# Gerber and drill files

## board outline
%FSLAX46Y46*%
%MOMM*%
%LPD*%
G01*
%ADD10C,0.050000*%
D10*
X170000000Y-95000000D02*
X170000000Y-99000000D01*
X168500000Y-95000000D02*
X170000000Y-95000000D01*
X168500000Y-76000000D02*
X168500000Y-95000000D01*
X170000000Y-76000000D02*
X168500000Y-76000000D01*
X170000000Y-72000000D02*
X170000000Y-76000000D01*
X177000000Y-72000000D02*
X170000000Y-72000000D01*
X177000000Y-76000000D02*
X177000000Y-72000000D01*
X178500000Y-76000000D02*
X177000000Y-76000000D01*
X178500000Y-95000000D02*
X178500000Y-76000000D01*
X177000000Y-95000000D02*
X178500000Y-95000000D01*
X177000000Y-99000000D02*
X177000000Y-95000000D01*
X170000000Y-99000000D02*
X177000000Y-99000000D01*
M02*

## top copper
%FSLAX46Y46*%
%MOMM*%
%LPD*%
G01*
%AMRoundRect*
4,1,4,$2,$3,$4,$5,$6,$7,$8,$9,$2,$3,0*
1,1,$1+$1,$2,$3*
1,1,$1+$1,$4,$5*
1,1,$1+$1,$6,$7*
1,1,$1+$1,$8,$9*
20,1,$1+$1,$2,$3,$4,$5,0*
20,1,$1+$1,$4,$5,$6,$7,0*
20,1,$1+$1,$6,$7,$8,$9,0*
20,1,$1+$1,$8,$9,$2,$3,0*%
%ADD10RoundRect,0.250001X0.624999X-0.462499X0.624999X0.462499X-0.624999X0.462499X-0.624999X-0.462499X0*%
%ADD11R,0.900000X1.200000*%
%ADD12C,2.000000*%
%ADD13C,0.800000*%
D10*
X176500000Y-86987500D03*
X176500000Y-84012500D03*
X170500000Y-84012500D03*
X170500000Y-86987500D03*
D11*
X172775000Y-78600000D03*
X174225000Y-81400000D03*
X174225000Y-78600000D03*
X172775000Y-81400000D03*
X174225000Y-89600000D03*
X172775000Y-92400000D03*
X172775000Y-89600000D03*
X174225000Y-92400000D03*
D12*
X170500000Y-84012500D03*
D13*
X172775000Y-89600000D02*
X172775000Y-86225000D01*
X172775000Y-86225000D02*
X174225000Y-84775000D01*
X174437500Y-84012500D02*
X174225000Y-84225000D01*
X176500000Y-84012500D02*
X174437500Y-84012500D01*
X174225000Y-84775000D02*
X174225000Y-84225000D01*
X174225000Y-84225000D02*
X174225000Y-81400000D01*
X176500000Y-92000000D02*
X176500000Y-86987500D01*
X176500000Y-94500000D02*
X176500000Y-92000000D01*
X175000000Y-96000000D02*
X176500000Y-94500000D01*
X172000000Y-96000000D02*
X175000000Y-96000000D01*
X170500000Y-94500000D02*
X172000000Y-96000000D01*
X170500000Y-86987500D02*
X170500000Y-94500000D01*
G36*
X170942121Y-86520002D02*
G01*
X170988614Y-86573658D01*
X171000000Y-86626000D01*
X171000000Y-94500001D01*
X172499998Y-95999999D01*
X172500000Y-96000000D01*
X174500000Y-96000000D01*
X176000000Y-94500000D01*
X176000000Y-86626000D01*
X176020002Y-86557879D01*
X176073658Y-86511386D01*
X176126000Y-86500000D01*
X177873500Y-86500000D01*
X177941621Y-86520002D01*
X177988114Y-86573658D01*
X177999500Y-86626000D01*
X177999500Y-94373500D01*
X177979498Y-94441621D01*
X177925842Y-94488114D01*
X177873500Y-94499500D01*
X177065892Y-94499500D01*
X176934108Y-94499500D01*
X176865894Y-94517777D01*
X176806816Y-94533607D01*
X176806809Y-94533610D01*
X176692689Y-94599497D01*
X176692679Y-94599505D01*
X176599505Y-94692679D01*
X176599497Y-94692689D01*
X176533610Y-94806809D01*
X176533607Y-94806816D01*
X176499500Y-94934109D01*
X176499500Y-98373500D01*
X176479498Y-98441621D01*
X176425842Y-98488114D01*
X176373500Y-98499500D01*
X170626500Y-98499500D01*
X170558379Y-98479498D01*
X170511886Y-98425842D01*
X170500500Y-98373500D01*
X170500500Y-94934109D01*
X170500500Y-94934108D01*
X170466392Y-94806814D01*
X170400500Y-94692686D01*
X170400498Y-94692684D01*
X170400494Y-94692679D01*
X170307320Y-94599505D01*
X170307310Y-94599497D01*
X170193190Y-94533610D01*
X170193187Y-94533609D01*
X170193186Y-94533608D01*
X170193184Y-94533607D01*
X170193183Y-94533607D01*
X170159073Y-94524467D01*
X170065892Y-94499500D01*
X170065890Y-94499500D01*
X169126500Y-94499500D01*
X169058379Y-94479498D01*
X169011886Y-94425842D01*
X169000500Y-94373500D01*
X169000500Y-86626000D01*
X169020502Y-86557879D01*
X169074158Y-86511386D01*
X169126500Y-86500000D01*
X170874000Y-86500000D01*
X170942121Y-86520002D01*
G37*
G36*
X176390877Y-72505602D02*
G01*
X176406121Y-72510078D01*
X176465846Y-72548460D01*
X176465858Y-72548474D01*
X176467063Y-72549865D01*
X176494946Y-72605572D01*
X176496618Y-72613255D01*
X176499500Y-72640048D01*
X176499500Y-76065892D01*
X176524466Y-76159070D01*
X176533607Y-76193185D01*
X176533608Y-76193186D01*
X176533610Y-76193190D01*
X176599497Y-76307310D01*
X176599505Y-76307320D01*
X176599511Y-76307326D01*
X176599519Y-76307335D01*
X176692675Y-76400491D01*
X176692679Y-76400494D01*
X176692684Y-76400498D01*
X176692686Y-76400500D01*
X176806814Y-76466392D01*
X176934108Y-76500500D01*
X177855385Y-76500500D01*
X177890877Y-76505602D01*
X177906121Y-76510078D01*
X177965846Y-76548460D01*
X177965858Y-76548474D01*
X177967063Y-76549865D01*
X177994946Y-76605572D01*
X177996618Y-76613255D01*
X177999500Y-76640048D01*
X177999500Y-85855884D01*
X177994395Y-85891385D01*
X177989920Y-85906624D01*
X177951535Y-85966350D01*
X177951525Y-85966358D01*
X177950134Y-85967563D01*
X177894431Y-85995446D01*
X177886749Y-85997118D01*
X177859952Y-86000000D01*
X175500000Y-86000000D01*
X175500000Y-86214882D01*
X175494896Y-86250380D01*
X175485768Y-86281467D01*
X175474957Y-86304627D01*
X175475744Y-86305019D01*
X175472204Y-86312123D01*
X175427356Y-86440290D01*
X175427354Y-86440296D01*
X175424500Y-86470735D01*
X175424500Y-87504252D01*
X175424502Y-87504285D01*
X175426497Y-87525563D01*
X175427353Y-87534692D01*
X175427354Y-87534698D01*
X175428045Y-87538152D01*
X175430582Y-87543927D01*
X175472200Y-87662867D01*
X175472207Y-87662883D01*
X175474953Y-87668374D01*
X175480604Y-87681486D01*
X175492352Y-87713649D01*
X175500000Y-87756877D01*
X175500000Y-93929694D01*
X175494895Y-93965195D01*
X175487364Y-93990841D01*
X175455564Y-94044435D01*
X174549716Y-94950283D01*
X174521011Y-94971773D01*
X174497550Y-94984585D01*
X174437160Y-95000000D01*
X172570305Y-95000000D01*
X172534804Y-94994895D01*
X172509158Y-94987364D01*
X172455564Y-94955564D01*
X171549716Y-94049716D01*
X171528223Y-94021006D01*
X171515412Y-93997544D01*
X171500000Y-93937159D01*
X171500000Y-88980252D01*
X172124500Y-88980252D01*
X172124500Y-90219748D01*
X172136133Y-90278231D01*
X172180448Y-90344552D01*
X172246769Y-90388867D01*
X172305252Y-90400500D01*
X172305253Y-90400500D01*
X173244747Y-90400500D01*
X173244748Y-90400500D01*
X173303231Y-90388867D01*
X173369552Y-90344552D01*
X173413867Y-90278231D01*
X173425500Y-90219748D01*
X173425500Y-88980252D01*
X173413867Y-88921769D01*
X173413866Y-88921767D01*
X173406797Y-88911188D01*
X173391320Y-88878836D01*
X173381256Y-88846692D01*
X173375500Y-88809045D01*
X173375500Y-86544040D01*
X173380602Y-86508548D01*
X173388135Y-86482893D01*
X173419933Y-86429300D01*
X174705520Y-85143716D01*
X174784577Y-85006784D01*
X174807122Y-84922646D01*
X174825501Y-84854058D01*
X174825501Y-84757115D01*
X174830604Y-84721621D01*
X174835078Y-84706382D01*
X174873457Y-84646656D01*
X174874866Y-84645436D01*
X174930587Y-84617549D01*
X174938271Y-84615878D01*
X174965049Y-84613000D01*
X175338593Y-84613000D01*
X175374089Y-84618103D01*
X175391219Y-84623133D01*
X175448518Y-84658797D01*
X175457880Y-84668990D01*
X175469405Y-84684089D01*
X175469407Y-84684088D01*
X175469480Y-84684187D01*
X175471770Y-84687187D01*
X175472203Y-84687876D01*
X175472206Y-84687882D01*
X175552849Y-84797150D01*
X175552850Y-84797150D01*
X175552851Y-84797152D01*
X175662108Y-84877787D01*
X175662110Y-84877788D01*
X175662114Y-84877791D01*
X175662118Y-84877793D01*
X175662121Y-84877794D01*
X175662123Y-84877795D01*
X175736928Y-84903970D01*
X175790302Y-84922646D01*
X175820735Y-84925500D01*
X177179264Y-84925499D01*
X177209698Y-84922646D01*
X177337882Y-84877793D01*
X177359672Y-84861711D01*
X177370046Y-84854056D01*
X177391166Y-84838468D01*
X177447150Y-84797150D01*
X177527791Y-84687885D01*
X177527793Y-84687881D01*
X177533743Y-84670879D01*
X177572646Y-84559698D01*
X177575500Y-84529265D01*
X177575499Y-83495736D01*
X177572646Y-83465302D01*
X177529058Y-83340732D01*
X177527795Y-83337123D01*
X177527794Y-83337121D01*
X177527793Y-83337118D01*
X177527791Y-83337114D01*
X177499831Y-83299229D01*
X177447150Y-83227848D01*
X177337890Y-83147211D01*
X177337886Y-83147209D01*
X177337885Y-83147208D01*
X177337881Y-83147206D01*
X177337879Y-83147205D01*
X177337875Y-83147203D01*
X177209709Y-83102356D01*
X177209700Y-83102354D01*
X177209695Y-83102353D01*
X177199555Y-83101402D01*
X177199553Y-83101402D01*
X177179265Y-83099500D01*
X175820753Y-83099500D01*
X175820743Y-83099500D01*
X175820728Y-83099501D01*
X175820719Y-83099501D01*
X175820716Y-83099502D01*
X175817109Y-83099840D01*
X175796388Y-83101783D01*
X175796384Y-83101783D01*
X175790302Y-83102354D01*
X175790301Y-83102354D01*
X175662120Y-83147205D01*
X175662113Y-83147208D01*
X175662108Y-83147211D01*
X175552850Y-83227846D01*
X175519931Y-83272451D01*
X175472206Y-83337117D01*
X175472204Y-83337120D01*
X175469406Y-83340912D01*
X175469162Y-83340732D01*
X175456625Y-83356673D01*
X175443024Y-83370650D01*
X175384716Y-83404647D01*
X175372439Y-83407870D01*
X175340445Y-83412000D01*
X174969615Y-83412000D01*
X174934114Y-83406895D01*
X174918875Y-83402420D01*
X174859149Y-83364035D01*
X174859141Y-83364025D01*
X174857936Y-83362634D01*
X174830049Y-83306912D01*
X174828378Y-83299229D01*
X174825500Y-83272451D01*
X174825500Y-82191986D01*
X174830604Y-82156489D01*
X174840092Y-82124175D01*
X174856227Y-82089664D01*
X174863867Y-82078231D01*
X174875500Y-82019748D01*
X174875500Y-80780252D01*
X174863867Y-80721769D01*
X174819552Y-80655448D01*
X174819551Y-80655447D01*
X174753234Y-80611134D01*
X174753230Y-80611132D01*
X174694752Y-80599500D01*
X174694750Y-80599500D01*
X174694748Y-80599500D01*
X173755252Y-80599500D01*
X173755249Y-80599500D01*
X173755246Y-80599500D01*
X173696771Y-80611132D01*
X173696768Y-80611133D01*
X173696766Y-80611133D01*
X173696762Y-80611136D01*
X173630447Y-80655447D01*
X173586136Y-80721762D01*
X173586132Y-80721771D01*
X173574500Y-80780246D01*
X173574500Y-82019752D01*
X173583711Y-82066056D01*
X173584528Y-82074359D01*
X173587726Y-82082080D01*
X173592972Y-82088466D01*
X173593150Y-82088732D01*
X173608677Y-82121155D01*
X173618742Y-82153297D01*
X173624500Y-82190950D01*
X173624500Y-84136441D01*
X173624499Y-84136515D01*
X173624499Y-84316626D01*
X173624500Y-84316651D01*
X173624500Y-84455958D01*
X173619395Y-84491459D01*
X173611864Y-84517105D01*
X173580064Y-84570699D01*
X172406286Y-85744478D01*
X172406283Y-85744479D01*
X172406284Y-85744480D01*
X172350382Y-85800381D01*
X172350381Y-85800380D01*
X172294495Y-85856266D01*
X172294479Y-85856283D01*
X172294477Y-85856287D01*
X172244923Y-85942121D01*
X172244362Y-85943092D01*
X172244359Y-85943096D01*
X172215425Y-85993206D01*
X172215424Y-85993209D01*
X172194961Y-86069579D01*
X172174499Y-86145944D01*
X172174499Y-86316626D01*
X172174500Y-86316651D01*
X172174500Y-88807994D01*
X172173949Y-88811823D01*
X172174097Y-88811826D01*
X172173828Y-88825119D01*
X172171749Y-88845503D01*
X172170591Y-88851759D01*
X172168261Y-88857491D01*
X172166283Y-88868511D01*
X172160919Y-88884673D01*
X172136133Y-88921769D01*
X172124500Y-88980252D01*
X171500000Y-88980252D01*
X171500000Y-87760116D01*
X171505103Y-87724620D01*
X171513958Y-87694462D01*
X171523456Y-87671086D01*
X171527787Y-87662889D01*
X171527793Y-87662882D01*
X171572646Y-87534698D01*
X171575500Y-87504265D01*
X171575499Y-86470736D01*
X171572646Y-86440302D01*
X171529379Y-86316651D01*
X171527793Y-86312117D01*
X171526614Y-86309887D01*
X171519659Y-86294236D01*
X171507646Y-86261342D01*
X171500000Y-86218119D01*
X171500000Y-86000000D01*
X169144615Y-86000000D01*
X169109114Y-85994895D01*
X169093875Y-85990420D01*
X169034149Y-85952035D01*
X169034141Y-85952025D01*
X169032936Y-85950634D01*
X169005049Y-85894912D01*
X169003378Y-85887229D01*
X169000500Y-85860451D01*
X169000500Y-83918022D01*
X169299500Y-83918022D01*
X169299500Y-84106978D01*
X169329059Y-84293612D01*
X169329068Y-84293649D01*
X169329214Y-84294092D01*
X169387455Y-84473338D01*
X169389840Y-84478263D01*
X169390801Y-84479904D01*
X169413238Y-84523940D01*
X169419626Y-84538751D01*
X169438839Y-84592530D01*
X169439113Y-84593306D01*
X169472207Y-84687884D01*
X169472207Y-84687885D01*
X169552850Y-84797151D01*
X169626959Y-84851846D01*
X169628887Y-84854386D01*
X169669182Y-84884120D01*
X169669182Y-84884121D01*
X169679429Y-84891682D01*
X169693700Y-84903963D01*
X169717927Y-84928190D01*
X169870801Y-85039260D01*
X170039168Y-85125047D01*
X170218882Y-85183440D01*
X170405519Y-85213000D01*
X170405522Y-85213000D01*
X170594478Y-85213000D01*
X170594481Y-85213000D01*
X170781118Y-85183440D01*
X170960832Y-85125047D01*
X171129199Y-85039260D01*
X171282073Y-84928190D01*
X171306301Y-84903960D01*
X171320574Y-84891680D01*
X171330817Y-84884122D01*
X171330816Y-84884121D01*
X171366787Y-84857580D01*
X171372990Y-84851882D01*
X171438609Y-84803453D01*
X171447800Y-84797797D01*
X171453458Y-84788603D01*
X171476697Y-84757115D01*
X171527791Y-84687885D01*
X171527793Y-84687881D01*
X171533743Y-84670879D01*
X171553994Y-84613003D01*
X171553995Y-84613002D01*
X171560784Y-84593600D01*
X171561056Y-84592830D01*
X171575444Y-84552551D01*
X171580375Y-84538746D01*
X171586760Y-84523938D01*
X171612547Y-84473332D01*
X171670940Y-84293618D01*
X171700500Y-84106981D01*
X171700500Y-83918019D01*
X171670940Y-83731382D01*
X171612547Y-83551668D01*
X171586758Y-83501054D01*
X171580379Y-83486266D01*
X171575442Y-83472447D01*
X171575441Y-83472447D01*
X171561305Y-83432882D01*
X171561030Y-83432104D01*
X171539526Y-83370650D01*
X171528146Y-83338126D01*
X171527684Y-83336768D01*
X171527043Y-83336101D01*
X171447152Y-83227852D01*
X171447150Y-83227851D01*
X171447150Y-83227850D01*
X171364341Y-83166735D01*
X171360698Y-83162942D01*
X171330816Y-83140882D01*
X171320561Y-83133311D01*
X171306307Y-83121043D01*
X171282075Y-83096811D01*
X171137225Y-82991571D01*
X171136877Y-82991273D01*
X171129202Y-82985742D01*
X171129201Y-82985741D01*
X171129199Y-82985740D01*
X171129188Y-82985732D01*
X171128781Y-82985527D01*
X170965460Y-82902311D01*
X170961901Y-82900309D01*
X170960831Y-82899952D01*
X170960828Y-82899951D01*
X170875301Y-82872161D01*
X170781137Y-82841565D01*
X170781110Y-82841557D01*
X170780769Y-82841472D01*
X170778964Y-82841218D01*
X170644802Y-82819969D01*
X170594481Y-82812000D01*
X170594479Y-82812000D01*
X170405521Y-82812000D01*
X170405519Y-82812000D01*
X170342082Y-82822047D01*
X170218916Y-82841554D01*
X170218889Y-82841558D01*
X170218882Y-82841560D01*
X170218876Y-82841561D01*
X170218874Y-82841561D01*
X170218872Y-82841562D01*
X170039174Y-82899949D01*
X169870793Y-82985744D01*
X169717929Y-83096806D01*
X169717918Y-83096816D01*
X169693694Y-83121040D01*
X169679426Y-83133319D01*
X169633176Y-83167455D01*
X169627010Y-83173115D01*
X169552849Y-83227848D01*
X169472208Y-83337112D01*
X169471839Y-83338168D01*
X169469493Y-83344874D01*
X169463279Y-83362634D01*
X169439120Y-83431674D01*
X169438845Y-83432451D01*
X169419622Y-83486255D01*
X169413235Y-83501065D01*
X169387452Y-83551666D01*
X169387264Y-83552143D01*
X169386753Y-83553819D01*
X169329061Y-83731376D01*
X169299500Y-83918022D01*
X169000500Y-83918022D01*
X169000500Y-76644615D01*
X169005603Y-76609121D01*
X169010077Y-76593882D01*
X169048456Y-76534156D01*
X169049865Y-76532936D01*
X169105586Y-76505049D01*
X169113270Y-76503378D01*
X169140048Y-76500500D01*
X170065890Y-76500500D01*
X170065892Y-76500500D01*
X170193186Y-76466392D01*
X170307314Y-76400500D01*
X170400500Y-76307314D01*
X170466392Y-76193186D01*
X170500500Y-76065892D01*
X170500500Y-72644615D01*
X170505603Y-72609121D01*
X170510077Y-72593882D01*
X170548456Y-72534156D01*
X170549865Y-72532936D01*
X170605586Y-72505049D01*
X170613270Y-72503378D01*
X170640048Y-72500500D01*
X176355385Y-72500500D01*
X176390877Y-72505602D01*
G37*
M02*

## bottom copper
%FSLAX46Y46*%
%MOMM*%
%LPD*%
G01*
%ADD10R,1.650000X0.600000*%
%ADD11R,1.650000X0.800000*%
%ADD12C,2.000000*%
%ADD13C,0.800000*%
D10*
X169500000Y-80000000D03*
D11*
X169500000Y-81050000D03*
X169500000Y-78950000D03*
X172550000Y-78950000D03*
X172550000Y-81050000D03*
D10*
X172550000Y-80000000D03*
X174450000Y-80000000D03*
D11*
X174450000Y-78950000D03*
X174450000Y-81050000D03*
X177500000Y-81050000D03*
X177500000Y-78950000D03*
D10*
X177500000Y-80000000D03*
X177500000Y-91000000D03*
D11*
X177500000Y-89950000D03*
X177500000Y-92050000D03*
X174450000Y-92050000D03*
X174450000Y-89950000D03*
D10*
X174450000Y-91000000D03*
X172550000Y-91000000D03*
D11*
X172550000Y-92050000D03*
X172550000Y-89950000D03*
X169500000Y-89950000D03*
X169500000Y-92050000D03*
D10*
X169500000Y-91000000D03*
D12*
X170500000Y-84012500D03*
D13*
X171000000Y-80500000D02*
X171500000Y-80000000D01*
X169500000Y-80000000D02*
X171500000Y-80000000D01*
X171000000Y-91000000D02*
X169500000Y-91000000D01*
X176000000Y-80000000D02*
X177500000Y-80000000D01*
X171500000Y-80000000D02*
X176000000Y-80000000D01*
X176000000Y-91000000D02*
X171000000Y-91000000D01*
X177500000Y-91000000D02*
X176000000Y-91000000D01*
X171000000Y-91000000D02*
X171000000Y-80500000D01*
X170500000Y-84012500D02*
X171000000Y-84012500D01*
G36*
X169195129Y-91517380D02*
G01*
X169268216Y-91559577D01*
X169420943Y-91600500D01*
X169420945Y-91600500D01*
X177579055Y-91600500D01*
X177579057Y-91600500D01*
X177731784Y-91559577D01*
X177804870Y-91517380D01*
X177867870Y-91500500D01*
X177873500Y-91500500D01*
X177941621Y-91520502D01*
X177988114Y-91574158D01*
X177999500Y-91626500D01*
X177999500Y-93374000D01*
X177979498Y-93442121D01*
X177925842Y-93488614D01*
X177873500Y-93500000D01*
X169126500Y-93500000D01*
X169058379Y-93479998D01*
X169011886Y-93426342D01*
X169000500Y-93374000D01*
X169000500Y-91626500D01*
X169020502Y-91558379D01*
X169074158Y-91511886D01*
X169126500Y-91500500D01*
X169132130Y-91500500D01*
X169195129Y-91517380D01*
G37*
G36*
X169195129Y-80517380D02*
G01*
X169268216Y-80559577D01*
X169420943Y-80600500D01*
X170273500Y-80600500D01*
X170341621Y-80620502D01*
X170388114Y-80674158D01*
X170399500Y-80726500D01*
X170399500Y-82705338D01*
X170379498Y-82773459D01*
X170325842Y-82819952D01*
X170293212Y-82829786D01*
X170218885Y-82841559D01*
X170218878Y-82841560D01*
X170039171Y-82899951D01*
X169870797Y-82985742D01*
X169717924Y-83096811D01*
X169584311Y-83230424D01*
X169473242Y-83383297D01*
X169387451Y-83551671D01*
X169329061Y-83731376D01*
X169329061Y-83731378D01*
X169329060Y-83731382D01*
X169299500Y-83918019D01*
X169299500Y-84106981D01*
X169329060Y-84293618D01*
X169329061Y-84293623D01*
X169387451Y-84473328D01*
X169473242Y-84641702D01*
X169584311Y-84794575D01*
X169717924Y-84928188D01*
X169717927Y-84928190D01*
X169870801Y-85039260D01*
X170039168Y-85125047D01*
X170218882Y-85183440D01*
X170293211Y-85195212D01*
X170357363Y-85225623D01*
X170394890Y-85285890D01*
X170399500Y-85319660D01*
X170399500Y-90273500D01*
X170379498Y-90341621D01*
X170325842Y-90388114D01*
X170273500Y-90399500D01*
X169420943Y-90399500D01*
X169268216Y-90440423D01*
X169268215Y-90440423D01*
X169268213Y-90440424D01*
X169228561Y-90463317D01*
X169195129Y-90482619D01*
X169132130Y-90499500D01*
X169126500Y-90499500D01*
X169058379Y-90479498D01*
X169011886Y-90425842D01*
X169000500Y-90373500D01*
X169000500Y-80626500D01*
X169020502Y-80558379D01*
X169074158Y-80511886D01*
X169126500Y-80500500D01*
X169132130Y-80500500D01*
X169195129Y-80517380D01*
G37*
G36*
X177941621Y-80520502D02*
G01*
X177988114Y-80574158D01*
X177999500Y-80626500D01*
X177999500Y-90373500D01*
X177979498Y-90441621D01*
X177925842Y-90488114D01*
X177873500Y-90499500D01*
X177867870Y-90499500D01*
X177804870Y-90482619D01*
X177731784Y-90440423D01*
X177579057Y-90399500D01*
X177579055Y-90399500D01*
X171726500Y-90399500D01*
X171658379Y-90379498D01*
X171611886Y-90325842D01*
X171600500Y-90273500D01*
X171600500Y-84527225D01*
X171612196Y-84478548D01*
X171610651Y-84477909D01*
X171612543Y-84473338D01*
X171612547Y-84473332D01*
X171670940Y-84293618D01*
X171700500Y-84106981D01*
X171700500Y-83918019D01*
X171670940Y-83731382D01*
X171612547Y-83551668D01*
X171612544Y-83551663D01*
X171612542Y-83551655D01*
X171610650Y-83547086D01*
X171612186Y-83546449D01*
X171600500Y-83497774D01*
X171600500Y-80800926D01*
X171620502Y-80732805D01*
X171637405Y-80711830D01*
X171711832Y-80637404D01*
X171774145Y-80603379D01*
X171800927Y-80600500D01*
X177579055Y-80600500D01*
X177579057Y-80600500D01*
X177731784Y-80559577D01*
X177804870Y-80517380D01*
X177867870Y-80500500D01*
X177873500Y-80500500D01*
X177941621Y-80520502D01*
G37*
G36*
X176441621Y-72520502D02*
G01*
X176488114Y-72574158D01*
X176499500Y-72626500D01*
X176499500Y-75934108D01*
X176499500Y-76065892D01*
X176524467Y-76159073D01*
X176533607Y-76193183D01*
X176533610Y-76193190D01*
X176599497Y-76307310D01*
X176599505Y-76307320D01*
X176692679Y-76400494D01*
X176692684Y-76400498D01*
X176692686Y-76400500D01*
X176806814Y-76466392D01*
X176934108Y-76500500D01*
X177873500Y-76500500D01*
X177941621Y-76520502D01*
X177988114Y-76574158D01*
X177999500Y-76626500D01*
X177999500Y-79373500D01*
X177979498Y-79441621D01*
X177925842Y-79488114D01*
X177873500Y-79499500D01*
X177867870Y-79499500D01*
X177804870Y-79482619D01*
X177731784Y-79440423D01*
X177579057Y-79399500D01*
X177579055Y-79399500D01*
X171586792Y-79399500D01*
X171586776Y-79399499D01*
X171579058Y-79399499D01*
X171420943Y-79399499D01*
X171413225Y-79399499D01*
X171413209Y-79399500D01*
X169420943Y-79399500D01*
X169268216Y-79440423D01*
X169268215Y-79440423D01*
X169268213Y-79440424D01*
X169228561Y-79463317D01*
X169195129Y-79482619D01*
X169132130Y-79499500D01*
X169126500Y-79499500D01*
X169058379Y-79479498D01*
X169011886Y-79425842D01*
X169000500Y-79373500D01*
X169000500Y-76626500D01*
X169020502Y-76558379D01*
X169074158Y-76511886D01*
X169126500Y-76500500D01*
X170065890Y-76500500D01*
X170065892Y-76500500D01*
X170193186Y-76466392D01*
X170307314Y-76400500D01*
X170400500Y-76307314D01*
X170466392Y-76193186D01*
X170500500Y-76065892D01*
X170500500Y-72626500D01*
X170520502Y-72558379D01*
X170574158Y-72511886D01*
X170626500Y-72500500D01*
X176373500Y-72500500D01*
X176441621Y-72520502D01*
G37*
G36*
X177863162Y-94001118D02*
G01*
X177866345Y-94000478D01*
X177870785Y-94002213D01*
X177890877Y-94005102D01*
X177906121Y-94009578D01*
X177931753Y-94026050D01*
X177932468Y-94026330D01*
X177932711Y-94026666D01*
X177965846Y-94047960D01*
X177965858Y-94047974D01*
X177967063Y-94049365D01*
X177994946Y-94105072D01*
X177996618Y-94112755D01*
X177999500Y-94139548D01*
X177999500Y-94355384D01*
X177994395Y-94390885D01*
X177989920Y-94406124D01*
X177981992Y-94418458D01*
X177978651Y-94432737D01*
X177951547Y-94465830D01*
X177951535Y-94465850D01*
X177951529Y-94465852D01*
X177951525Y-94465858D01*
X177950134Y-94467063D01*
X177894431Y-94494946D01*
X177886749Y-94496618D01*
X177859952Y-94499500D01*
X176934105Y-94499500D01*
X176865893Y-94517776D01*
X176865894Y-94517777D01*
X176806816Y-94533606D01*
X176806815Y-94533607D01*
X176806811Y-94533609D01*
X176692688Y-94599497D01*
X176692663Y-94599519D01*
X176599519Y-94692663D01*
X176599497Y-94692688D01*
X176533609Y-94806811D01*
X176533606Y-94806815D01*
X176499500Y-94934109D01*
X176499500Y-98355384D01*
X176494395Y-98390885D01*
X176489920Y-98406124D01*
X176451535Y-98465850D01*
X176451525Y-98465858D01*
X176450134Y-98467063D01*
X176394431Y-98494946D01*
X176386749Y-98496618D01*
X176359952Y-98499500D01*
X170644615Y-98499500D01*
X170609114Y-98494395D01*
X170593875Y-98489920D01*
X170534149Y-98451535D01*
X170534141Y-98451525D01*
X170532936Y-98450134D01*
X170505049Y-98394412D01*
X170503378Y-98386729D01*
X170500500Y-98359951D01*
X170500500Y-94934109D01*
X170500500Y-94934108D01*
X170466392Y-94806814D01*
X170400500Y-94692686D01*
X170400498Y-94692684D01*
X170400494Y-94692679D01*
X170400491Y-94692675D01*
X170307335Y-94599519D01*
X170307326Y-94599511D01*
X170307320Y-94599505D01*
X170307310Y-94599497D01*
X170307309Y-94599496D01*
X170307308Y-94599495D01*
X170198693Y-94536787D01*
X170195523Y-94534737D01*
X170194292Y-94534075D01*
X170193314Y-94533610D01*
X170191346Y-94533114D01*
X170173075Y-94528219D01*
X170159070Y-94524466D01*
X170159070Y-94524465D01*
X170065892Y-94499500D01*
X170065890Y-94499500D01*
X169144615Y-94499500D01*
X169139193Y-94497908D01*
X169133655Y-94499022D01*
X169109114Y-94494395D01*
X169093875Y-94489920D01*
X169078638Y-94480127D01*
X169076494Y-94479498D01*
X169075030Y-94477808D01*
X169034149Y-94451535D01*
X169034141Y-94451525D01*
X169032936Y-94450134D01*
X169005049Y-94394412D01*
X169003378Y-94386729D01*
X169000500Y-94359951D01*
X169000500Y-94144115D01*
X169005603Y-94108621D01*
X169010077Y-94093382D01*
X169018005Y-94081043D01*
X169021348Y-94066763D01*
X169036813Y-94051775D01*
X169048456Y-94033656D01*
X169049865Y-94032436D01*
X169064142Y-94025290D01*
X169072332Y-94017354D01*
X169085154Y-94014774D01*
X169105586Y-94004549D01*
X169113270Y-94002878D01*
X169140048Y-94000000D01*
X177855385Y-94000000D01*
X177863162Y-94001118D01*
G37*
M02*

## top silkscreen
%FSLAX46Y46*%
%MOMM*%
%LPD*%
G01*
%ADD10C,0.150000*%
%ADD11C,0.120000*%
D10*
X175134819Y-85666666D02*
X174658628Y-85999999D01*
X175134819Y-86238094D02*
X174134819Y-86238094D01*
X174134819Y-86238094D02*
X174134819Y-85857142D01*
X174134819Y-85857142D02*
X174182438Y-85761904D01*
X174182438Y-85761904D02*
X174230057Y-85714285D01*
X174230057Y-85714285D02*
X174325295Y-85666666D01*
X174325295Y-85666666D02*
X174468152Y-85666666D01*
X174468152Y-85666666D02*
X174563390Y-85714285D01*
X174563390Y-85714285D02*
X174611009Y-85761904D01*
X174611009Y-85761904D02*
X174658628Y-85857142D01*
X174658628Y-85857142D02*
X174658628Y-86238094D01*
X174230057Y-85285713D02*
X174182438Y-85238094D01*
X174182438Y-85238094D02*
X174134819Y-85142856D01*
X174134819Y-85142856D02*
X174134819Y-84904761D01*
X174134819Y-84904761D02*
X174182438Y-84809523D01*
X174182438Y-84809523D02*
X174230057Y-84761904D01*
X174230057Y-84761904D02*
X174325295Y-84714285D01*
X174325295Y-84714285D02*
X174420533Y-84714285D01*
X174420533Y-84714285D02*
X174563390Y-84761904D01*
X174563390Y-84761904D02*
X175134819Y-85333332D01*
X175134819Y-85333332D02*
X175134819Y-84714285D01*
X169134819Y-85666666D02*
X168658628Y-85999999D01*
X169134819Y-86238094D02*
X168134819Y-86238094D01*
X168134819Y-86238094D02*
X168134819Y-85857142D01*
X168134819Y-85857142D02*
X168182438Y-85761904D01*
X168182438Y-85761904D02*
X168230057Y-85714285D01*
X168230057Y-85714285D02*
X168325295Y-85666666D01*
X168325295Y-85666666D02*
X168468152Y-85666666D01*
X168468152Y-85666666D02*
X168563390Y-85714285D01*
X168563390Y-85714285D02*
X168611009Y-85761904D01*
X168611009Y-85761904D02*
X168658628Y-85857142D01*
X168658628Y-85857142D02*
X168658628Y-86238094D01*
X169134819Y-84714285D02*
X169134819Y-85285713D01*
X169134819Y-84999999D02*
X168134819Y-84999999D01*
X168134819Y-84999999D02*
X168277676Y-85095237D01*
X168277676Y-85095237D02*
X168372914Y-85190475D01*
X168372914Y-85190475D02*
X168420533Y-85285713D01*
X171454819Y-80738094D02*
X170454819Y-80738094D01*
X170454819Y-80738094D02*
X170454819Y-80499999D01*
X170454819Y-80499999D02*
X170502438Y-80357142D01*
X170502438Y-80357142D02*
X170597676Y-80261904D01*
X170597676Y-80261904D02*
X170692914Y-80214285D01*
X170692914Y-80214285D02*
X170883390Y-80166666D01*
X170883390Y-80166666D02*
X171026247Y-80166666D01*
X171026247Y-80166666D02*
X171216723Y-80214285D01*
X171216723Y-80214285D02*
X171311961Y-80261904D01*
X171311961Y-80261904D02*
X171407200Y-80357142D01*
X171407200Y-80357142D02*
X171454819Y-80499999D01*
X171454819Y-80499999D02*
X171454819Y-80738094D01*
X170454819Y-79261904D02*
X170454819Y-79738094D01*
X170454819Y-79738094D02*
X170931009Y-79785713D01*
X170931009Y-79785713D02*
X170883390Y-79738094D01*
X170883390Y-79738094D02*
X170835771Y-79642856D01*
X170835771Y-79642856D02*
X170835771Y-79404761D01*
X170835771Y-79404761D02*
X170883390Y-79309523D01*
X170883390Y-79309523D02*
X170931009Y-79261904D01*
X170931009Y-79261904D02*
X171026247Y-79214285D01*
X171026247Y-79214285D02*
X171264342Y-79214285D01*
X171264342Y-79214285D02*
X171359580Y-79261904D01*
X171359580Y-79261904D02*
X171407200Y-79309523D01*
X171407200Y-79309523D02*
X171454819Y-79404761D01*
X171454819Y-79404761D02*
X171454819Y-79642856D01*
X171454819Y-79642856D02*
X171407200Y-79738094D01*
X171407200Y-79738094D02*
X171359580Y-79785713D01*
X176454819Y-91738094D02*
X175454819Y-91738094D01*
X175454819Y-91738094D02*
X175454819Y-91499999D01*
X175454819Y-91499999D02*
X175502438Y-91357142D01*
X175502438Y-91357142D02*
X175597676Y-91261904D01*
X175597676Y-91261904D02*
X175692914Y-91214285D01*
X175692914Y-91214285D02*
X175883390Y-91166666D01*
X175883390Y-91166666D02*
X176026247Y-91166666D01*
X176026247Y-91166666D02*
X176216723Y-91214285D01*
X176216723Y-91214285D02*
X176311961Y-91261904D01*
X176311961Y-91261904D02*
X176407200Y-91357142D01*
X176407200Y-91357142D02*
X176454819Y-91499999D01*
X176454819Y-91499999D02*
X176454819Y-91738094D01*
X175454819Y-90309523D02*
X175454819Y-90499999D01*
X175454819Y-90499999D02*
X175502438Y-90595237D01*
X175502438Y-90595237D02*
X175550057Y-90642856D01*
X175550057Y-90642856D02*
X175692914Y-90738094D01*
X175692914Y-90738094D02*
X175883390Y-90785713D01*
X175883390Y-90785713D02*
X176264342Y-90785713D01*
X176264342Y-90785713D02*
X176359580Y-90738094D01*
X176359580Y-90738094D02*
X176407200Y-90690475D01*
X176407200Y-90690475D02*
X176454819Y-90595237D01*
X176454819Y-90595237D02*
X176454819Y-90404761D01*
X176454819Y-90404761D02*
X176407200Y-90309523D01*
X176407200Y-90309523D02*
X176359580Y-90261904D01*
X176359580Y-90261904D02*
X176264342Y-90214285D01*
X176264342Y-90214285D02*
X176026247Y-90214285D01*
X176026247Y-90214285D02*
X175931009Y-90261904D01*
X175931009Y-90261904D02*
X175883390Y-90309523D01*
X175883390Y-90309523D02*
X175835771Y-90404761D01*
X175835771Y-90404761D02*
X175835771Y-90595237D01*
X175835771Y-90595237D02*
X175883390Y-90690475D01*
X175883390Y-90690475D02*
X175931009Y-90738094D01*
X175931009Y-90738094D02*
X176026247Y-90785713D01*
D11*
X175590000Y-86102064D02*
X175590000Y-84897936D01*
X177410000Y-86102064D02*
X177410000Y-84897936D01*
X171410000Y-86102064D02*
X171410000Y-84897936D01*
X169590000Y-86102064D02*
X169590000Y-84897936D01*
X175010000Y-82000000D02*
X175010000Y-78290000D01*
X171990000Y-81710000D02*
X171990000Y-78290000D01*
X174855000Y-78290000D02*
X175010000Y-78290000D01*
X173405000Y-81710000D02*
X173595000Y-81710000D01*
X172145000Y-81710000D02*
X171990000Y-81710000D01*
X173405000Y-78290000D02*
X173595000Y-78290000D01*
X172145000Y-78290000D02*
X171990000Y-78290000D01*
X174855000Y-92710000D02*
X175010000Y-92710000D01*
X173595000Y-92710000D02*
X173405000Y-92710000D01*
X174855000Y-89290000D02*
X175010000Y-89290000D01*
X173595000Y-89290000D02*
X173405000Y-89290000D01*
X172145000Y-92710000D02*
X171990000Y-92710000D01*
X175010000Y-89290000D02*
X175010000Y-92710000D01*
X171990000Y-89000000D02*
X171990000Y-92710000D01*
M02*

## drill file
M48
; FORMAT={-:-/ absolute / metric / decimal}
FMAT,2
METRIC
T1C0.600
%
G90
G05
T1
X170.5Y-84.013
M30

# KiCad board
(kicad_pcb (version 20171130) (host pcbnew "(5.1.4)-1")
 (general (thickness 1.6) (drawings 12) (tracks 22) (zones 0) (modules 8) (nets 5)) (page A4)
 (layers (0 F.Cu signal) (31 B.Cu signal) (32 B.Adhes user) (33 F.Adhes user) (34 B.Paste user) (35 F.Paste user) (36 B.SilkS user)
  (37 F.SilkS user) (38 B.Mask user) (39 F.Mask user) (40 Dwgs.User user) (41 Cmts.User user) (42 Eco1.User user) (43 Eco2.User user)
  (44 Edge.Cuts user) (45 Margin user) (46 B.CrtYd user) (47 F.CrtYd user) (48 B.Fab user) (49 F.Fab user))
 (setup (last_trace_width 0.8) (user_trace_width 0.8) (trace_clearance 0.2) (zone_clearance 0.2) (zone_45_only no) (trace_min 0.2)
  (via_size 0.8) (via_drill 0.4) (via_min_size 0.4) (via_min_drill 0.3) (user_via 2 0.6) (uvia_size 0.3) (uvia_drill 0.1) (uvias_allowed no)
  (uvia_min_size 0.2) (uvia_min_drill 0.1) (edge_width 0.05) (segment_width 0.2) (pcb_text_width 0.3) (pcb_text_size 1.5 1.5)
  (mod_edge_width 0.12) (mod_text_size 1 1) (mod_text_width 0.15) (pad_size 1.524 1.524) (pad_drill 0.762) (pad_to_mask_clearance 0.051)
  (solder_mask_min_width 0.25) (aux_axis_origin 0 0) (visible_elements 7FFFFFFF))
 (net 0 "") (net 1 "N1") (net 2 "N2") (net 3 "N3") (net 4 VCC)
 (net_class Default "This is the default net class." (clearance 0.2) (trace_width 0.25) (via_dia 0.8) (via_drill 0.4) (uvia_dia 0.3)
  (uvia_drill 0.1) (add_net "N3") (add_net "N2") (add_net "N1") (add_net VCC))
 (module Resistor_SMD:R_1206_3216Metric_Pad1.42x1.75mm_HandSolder (layer F.Cu) (at 176.5 85.5 90)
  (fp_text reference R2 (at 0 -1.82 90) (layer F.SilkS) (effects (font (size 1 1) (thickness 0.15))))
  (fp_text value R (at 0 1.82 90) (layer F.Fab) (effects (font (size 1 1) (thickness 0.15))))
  (fp_line (start -0.602064 -0.91) (end 0.602064 -0.91) (layer F.SilkS) (width 0.12))
  (fp_line (start -0.602064 0.91) (end 0.602064 0.91) (layer F.SilkS) (width 0.12))
  (pad 1 smd roundrect (at -1.4875 0 90) (size 1.425 1.75) (layers F.Cu F.Paste F.Mask) (roundrect_rratio 0.175439) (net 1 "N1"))
  (pad 2 smd roundrect (at 1.4875 0 90) (size 1.425 1.75) (layers F.Cu F.Paste F.Mask) (roundrect_rratio 0.175439) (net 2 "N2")))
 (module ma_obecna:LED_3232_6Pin (layer B.Cu) (at 169.5 80)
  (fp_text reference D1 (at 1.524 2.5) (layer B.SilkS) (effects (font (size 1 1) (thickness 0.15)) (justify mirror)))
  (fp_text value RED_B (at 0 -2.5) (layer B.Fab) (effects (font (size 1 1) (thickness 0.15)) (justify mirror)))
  (pad 2 smd rect (at 0 0) (size 1.65 0.6) (layers B.Cu B.Paste B.Mask) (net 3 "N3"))
  (pad 1 smd rect (at 0 1.05) (size 1.65 0.8) (layers B.Cu B.Paste B.Mask) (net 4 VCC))
  (pad 3 smd rect (at 0 -1.05) (size 1.65 0.8) (layers B.Cu B.Paste B.Mask) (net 4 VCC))
  (pad 4 smd rect (at 3.05 -1.05) (size 1.65 0.8) (layers B.Cu B.Paste B.Mask) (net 4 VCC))
  (pad 6 smd rect (at 3.05 1.05) (size 1.65 0.8) (layers B.Cu B.Paste B.Mask) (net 4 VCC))
  (pad 5 smd rect (at 3.05 0) (size 1.65 0.6) (layers B.Cu B.Paste B.Mask) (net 3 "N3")))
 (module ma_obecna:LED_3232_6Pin (layer B.Cu) (at 177.5 80 180)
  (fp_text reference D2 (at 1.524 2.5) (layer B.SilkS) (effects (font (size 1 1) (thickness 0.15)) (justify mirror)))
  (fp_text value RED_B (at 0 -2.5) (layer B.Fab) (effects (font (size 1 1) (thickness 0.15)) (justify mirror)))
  (pad 5 smd rect (at 3.05 0 180) (size 1.65 0.6) (layers B.Cu B.Paste B.Mask) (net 3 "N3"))
  (pad 6 smd rect (at 3.05 1.05 180) (size 1.65 0.8) (layers B.Cu B.Paste B.Mask) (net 4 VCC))
  (pad 4 smd rect (at 3.05 -1.05 180) (size 1.65 0.8) (layers B.Cu B.Paste B.Mask) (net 4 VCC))
  (pad 3 smd rect (at 0 -1.05 180) (size 1.65 0.8) (layers B.Cu B.Paste B.Mask) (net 4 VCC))
  (pad 1 smd rect (at 0 1.05 180) (size 1.65 0.8) (layers B.Cu B.Paste B.Mask) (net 4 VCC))
  (pad 2 smd rect (at 0 0 180) (size 1.65 0.6) (layers B.Cu B.Paste B.Mask) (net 3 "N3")))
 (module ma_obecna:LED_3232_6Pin (layer B.Cu) (at 177.5 91 180)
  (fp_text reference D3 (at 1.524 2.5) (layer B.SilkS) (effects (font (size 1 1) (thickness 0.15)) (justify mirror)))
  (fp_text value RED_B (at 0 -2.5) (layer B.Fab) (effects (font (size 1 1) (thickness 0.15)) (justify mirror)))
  (pad 2 smd rect (at 0 0 180) (size 1.65 0.6) (layers B.Cu B.Paste B.Mask) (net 3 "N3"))
  (pad 1 smd rect (at 0 1.05 180) (size 1.65 0.8) (layers B.Cu B.Paste B.Mask) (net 4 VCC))
  (pad 3 smd rect (at 0 -1.05 180) (size 1.65 0.8) (layers B.Cu B.Paste B.Mask) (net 4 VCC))
  (pad 4 smd rect (at 3.05 -1.05 180) (size 1.65 0.8) (layers B.Cu B.Paste B.Mask) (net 4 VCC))
  (pad 6 smd rect (at 3.05 1.05 180) (size 1.65 0.8) (layers B.Cu B.Paste B.Mask) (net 4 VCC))
  (pad 5 smd rect (at 3.05 0 180) (size 1.65 0.6) (layers B.Cu B.Paste B.Mask) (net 3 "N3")))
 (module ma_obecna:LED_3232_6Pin (layer B.Cu) (at 169.5 91)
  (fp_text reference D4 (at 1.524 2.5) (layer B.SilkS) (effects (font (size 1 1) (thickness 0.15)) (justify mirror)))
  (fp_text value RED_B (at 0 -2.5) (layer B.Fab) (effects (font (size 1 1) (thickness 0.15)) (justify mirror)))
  (pad 5 smd rect (at 3.05 0) (size 1.65 0.6) (layers B.Cu B.Paste B.Mask) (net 3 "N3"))
  (pad 6 smd rect (at 3.05 1.05) (size 1.65 0.8) (layers B.Cu B.Paste B.Mask) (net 4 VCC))
  (pad 4 smd rect (at 3.05 -1.05) (size 1.65 0.8) (layers B.Cu B.Paste B.Mask) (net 4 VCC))
  (pad 3 smd rect (at 0 -1.05) (size 1.65 0.8) (layers B.Cu B.Paste B.Mask) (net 4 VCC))
  (pad 1 smd rect (at 0 1.05) (size 1.65 0.8) (layers B.Cu B.Paste B.Mask) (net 4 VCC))
  (pad 2 smd rect (at 0 0) (size 1.65 0.6) (layers B.Cu B.Paste B.Mask) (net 3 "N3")))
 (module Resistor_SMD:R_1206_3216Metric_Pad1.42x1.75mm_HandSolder (layer F.Cu) (at 170.5 85.5 90)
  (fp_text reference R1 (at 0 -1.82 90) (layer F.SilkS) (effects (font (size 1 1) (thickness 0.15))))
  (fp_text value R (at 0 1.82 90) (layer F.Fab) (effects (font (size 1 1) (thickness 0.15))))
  (fp_line (start -0.602064 0.91) (end 0.602064 0.91) (layer F.SilkS) (width 0.12))
  (fp_line (start -0.602064 -0.91) (end 0.602064 -0.91) (layer F.SilkS) (width 0.12))
  (pad 2 smd roundrect (at 1.4875 0 90) (size 1.425 1.75) (layers F.Cu F.Paste F.Mask) (roundrect_rratio 0.175439) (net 3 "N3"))
  (pad 1 smd roundrect (at -1.4875 0 90) (size 1.425 1.75) (layers F.Cu F.Paste F.Mask) (roundrect_rratio 0.175439) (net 1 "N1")))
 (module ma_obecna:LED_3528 (layer F.Cu) (at 173.5 80 90)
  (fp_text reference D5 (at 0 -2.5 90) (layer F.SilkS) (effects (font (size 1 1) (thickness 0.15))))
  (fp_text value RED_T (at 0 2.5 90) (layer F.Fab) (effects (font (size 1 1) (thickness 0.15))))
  (fp_line (start -2 1.51) (end 1.71 1.51) (layer F.SilkS) (width 0.12))
  (fp_line (start -1.71 -1.51) (end 1.71 -1.51) (layer F.SilkS) (width 0.12))
  (fp_line (start 1.71 1.355) (end 1.71 1.51) (layer F.SilkS) (width 0.12))
  (fp_line (start -1.71 -0.095) (end -1.71 0.095) (layer F.SilkS) (width 0.12))
  (fp_line (start -1.71 -1.355) (end -1.71 -1.51) (layer F.SilkS) (width 0.12))
  (fp_line (start 1.71 -0.095) (end 1.71 0.095) (layer F.SilkS) (width 0.12))
  (fp_line (start 1.71 -1.355) (end 1.71 -1.51) (layer F.SilkS) (width 0.12))
  (pad 3 smd rect (at 1.4 -0.725 90) (size 1.2 0.9) (layers F.Cu F.Paste F.Mask) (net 4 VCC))
  (pad 1 smd rect (at -1.4 0.725 90) (size 1.2 0.9) (layers F.Cu F.Paste F.Mask) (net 2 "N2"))
  (pad 2 smd rect (at 1.4 0.725 90) (size 1.2 0.9) (layers F.Cu F.Paste F.Mask) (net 4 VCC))
  (pad 4 smd rect (at -1.4 -0.725 90) (size 1.2 0.9) (layers F.Cu F.Paste F.Mask) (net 4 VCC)))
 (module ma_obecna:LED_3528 (layer F.Cu) (at 173.5 91 270)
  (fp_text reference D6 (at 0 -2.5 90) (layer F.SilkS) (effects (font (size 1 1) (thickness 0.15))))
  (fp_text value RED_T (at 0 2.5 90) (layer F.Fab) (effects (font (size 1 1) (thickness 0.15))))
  (fp_line (start 1.71 -1.355) (end 1.71 -1.51) (layer F.SilkS) (width 0.12))
  (fp_line (start 1.71 -0.095) (end 1.71 0.095) (layer F.SilkS) (width 0.12))
  (fp_line (start -1.71 -1.355) (end -1.71 -1.51) (layer F.SilkS) (width 0.12))
  (fp_line (start -1.71 -0.095) (end -1.71 0.095) (layer F.SilkS) (width 0.12))
  (fp_line (start 1.71 1.355) (end 1.71 1.51) (layer F.SilkS) (width 0.12))
  (fp_line (start -1.71 -1.51) (end 1.71 -1.51) (layer F.SilkS) (width 0.12))
  (fp_line (start -2 1.51) (end 1.71 1.51) (layer F.SilkS) (width 0.12))
  (pad 4 smd rect (at -1.4 -0.725 270) (size 1.2 0.9) (layers F.Cu F.Paste F.Mask) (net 4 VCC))
  (pad 2 smd rect (at 1.4 0.725 270) (size 1.2 0.9) (layers F.Cu F.Paste F.Mask) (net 4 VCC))
  (pad 1 smd rect (at -1.4 0.725 270) (size 1.2 0.9) (layers F.Cu F.Paste F.Mask) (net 2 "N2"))
  (pad 3 smd rect (at 1.4 -0.725 270) (size 1.2 0.9) (layers F.Cu F.Paste F.Mask) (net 4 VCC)))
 (gr_line (start 170 95) (end 170 99) (layer Edge.Cuts) (width 0.05))
 (gr_line (start 168.5 95) (end 170 95) (layer Edge.Cuts) (width 0.05))
 (gr_line (start 168.5 76) (end 168.5 95) (layer Edge.Cuts) (width 0.05))
 (gr_line (start 170 76) (end 168.5 76) (layer Edge.Cuts) (width 0.05))
 (gr_line (start 170 72) (end 170 76) (layer Edge.Cuts) (width 0.05))
 (gr_line (start 177 72) (end 170 72) (layer Edge.Cuts) (width 0.05))
 (gr_line (start 177 76) (end 177 72) (layer Edge.Cuts) (width 0.05))
 (gr_line (start 178.5 76) (end 177 76) (layer Edge.Cuts) (width 0.05))
 (gr_line (start 178.5 95) (end 178.5 76) (layer Edge.Cuts) (width 0.05))
 (gr_line (start 177 95) (end 178.5 95) (layer Edge.Cuts) (width 0.05))
 (gr_line (start 177 99) (end 177 95) (layer Edge.Cuts) (width 0.05))
 (gr_line (start 170 99) (end 177 99) (layer Edge.Cuts) (width 0.05))
 (segment (start 172.775 89.6) (end 172.775 86.225) (width 0.8) (layer F.Cu) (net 2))
 (segment (start 172.775 86.225) (end 174.225 84.775) (width 0.8) (layer F.Cu) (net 2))
 (segment (start 174.4375 84.0125) (end 174.225 84.225) (width 0.8) (layer F.Cu) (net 2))
 (segment (start 176.5 84.0125) (end 174.4375 84.0125) (width 0.8) (layer F.Cu) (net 2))
 (segment (start 174.225 84.775) (end 174.225 84.225) (width 0.8) (layer F.Cu) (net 2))
 (segment (start 174.225 84.225) (end 174.225 81.4) (width 0.8) (layer F.Cu) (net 2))
 (segment (start 176.5 92) (end 176.5 86.9875) (width 0.8) (layer F.Cu) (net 1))
 (segment (start 176.5 94.5) (end 176.5 92) (width 0.8) (layer F.Cu) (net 1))
 (segment (start 175 96) (end 176.5 94.5) (width 0.8) (layer F.Cu) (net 1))
 (segment (start 172 96) (end 175 96) (width 0.8) (layer F.Cu) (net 1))
 (segment (start 170.5 94.5) (end 172 96) (width 0.8) (layer F.Cu) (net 1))
 (segment (start 170.5 86.9875) (end 170.5 94.5) (width 0.8) (layer F.Cu) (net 1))
 (segment (start 171 80.5) (end 171.5 80) (width 0.8) (layer B.Cu) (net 3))
 (segment (start 169.5 80) (end 171.5 80) (width 0.8) (layer B.Cu) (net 3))
 (segment (start 171 91) (end 169.5 91) (width 0.8) (layer B.Cu) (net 3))
 (segment (start 176 80) (end 177.5 80) (width 0.8) (layer B.Cu) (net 3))
 (segment (start 171.5 80) (end 176 80) (width 0.8) (layer B.Cu) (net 3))
 (segment (start 176 91) (end 171 91) (width 0.8) (layer B.Cu) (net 3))
 (segment (start 177.5 91) (end 176 91) (width 0.8) (layer B.Cu) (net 3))
 (segment (start 171 91) (end 171 80.5) (width 0.8) (layer B.Cu) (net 3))
 (via (at 170.5 84.0125) (size 2) (drill 0.6) (layers F.Cu B.Cu) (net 3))
 (segment (start 170.5 84.0125) (end 171 84.0125) (width 0.8) (layer B.Cu) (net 3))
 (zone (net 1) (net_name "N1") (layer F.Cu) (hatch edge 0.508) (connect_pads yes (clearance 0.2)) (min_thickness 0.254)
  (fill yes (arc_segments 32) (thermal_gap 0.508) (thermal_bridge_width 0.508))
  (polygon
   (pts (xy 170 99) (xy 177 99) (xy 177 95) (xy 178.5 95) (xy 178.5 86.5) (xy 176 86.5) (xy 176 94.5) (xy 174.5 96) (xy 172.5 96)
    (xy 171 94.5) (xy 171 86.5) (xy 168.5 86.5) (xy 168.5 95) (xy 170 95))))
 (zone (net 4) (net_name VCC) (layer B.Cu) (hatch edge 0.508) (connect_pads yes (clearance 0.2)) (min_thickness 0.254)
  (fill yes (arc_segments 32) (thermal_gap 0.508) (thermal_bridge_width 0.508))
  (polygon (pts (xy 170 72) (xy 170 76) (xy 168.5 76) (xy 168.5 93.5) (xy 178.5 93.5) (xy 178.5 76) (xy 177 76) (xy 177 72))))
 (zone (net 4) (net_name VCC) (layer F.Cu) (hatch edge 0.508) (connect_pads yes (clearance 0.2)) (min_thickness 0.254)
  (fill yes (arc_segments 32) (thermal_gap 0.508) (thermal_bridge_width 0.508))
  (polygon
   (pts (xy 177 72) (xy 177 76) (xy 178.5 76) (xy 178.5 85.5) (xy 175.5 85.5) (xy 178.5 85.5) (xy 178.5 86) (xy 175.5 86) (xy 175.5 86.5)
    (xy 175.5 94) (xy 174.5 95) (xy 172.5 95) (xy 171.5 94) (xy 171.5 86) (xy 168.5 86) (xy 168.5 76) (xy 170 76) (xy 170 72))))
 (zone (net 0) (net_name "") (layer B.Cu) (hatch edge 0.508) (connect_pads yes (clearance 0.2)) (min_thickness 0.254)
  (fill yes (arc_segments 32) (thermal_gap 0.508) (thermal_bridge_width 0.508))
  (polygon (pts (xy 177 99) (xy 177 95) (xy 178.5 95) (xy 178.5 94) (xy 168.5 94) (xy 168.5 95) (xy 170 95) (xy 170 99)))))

